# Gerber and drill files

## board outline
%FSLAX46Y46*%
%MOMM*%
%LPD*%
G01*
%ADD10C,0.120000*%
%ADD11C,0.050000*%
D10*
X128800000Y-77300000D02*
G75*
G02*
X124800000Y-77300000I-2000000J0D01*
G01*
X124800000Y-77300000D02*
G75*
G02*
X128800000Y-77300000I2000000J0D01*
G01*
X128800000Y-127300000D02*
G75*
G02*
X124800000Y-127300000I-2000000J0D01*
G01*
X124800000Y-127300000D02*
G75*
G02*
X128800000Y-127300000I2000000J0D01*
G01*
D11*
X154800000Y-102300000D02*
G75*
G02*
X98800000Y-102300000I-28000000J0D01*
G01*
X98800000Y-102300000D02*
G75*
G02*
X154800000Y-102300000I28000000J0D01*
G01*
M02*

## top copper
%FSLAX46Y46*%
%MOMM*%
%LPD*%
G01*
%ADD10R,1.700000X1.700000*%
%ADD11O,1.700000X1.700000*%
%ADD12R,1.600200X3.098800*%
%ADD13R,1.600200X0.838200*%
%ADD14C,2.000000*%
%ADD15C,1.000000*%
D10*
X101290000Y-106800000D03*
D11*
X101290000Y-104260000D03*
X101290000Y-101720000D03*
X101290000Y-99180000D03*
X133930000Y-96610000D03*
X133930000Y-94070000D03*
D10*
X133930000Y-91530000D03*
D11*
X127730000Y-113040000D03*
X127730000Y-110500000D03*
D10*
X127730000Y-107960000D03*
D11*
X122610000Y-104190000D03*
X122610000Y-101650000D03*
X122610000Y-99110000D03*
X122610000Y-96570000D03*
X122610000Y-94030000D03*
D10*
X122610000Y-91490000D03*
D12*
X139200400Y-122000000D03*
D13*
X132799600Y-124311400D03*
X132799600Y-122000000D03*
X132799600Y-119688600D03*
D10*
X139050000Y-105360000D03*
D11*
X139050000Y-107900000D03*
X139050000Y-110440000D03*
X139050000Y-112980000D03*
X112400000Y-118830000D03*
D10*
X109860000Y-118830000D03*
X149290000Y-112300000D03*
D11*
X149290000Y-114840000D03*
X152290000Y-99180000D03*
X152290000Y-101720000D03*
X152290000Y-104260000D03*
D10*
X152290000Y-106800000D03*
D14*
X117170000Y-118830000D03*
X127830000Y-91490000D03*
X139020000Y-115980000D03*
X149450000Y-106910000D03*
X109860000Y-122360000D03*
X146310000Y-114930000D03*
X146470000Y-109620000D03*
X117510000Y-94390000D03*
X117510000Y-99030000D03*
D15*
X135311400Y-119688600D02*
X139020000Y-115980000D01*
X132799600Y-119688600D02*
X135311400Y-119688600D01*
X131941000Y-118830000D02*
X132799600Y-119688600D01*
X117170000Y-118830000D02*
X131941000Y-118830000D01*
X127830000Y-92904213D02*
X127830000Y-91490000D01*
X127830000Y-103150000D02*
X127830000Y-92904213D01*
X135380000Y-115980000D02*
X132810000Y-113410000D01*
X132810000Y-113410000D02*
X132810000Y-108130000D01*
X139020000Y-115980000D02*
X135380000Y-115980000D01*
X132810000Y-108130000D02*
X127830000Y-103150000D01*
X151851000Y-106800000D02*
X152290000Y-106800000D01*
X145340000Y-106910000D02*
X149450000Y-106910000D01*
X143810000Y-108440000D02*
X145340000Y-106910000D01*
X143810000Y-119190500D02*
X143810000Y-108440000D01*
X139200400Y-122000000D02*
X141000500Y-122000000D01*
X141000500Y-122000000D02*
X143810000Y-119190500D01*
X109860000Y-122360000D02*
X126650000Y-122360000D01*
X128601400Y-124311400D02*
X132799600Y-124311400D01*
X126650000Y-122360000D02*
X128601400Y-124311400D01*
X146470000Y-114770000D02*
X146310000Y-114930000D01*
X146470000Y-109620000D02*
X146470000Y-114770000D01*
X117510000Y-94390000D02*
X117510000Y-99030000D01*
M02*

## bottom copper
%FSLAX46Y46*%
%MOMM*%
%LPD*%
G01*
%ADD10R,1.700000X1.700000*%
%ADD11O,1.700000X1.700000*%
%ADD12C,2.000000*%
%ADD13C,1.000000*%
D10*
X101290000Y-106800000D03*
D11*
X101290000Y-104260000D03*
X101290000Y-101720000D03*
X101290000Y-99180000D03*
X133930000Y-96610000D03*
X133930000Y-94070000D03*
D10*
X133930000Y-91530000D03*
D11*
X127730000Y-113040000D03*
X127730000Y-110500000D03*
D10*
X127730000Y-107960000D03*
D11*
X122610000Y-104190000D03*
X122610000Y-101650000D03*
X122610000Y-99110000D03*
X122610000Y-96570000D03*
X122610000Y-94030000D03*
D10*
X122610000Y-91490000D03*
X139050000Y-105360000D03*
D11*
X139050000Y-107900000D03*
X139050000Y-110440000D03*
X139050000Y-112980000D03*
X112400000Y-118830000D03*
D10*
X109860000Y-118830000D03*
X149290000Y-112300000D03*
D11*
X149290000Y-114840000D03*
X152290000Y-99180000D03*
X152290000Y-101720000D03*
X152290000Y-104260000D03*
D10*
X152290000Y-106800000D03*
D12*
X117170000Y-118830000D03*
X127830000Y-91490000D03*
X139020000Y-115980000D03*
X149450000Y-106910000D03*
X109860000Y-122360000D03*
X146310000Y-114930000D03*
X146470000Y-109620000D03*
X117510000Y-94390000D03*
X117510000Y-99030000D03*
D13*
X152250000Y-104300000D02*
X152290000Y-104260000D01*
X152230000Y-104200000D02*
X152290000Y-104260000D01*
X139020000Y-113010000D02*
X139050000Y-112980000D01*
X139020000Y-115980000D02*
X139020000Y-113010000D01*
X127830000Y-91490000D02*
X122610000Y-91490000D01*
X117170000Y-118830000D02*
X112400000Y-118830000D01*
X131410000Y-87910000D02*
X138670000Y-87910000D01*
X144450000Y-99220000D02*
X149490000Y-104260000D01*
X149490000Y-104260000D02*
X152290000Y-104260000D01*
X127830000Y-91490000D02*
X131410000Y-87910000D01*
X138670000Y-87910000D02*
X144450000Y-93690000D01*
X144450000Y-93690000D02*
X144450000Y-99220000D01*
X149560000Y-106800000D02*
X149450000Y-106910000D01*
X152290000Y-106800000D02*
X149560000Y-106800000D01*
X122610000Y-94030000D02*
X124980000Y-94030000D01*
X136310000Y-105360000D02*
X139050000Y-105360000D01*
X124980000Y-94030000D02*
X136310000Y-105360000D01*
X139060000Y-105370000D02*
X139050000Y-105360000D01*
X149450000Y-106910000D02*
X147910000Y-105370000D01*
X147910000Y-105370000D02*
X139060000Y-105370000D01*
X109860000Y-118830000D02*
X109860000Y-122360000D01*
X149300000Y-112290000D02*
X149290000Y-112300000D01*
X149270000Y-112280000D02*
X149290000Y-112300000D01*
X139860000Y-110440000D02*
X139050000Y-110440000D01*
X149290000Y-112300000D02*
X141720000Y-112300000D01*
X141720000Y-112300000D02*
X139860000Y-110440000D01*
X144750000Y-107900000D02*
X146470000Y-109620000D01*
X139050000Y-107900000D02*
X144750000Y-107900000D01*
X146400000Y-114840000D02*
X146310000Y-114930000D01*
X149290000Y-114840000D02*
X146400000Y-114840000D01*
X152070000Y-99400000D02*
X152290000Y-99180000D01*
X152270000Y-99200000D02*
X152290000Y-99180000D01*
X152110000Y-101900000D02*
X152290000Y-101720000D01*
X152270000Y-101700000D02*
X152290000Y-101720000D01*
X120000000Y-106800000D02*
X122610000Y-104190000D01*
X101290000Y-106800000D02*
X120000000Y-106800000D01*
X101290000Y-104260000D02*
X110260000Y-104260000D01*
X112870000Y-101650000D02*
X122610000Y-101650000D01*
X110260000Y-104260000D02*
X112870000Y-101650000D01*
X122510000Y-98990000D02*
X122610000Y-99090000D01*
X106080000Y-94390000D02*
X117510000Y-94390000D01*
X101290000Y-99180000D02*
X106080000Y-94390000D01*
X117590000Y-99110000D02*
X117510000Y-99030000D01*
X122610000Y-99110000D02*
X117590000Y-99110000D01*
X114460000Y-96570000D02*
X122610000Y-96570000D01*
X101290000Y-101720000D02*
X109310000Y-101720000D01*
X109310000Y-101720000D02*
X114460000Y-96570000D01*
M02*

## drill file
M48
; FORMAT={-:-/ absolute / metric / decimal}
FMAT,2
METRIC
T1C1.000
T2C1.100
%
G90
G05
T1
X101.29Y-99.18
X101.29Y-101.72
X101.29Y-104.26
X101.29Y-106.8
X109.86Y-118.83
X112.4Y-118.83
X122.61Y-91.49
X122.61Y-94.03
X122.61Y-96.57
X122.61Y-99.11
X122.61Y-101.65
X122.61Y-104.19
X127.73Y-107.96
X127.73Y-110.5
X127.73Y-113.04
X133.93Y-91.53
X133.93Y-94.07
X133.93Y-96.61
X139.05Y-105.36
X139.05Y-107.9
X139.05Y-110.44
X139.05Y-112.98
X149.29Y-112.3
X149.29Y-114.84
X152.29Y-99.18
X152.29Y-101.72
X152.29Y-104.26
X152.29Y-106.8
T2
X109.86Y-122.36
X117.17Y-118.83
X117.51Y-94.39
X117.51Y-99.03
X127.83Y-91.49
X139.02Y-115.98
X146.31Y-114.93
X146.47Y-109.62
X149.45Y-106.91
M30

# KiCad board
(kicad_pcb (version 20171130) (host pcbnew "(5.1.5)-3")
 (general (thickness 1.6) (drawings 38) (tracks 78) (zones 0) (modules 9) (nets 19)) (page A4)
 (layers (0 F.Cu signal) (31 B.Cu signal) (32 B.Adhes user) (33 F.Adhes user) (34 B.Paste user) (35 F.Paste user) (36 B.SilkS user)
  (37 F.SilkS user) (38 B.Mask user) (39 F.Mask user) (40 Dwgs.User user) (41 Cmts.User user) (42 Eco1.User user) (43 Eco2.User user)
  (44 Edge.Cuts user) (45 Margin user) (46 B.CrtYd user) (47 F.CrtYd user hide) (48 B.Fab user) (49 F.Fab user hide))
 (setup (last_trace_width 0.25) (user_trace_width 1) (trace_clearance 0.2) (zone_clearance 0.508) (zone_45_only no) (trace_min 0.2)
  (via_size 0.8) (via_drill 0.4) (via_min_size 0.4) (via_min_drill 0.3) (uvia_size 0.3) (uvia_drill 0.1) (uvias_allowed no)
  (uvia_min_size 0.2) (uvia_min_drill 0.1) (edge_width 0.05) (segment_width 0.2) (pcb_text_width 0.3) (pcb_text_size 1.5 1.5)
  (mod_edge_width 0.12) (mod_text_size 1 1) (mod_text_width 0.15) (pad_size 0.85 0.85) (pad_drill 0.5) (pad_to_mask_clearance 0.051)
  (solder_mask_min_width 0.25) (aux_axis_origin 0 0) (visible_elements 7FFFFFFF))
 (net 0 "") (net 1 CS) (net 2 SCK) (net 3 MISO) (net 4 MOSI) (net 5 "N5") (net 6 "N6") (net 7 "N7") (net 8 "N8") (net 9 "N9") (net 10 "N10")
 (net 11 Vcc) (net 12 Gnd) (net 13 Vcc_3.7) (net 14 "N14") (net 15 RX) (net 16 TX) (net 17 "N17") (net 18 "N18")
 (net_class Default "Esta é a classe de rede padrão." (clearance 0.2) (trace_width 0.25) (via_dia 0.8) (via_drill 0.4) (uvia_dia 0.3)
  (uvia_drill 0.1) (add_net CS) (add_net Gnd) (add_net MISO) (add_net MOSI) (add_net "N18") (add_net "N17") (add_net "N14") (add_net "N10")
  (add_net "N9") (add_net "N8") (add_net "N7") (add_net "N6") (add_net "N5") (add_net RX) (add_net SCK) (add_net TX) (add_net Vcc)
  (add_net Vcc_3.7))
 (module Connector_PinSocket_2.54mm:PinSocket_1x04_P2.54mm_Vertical (layer F.Cu) (at 101.29 106.8 180)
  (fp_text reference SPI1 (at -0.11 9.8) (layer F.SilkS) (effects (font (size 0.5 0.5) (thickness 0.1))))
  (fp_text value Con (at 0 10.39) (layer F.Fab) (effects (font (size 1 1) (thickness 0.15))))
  (pad 1 thru_hole rect (at 0 0 180) (size 1.7 1.7) (drill 1) (layers *.Cu *.Mask) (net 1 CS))
  (pad 2 thru_hole oval (at 0 2.54 180) (size 1.7 1.7) (drill 1) (layers *.Cu *.Mask) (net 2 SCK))
  (pad 3 thru_hole oval (at 0 5.08 180) (size 1.7 1.7) (drill 1) (layers *.Cu *.Mask) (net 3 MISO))
  (pad 4 thru_hole oval (at 0 7.62 180) (size 1.7 1.7) (drill 1) (layers *.Cu *.Mask) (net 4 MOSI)))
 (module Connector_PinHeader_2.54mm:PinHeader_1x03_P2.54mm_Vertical (layer F.Cu) (at 133.93 91.53)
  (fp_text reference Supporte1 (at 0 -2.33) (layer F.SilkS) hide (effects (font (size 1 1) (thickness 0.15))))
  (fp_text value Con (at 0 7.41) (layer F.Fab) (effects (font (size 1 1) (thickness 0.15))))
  (pad 3 thru_hole oval (at 0 5.08) (size 1.7 1.7) (drill 1) (layers *.Cu *.Mask) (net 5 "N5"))
  (pad 2 thru_hole oval (at 0 2.54) (size 1.7 1.7) (drill 1) (layers *.Cu *.Mask) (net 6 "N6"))
  (pad 1 thru_hole rect (at 0 0) (size 1.7 1.7) (drill 1) (layers *.Cu *.Mask) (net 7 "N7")))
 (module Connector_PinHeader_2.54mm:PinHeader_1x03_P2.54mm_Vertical (layer F.Cu) (at 127.73 107.96)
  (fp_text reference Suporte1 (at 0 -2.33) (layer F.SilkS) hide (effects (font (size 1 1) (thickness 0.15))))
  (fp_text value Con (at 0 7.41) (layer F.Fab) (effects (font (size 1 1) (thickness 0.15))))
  (pad 3 thru_hole oval (at 0 5.08) (size 1.7 1.7) (drill 1) (layers *.Cu *.Mask) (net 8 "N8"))
  (pad 2 thru_hole oval (at 0 2.54) (size 1.7 1.7) (drill 1) (layers *.Cu *.Mask) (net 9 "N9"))
  (pad 1 thru_hole rect (at 0 0) (size 1.7 1.7) (drill 1) (layers *.Cu *.Mask) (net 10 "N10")))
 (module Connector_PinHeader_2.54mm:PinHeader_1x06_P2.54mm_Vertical (layer F.Cu) (at 122.61 91.49)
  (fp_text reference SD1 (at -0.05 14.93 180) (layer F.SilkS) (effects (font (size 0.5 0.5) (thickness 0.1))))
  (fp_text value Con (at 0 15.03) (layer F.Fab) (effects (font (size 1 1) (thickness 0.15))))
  (pad 6 thru_hole oval (at 0 12.7) (size 1.7 1.7) (drill 1) (layers *.Cu *.Mask) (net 1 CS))
  (pad 5 thru_hole oval (at 0 10.16) (size 1.7 1.7) (drill 1) (layers *.Cu *.Mask) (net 2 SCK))
  (pad 4 thru_hole oval (at 0 7.62) (size 1.7 1.7) (drill 1) (layers *.Cu *.Mask) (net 4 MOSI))
  (pad 3 thru_hole oval (at 0 5.08) (size 1.7 1.7) (drill 1) (layers *.Cu *.Mask) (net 3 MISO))
  (pad 2 thru_hole oval (at 0 2.54) (size 1.7 1.7) (drill 1) (layers *.Cu *.Mask) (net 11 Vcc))
  (pad 1 thru_hole rect (at 0 0) (size 1.7 1.7) (drill 1) (layers *.Cu *.Mask) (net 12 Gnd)))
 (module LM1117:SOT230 (layer F.Cu) (at 136 122)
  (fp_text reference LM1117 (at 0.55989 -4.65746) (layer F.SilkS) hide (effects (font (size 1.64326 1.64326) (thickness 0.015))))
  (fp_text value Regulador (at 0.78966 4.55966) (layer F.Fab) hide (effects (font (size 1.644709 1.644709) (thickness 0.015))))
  (pad 4 smd rect (at 3.2004 0) (size 1.6002 3.0988) (layers F.Cu F.Paste F.Mask) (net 11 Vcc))
  (pad 3 smd rect (at -3.2004 2.3114) (size 1.6002 0.8382) (layers F.Cu F.Paste F.Mask) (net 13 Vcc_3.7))
  (pad 2 smd rect (at -3.2004 0) (size 1.6002 0.8382) (layers F.Cu F.Paste F.Mask) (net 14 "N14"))
  (pad 1 smd rect (at -3.2004 -2.3114) (size 1.6002 0.8382) (layers F.Cu F.Paste F.Mask) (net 12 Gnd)))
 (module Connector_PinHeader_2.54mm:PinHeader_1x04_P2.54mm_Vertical (layer F.Cu) (at 139.05 105.36)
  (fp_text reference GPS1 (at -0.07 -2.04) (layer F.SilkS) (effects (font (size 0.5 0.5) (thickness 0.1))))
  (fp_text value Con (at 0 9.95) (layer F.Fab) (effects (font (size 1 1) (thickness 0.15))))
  (pad 1 thru_hole rect (at 0 0) (size 1.7 1.7) (drill 1) (layers *.Cu *.Mask) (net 11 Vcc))
  (pad 2 thru_hole oval (at 0 2.54) (size 1.7 1.7) (drill 1) (layers *.Cu *.Mask) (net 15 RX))
  (pad 3 thru_hole oval (at 0 5.08) (size 1.7 1.7) (drill 1) (layers *.Cu *.Mask) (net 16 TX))
  (pad 4 thru_hole oval (at 0 7.62) (size 1.7 1.7) (drill 1) (layers *.Cu *.Mask) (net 12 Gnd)))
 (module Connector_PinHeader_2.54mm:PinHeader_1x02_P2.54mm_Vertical (layer F.Cu) (at 109.86 118.83 90)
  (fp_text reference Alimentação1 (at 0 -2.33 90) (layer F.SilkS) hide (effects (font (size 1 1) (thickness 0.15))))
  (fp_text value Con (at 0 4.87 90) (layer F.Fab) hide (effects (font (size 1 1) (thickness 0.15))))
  (pad 2 thru_hole oval (at 0 2.54 90) (size 1.7 1.7) (drill 1) (layers *.Cu *.Mask) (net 12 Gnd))
  (pad 1 thru_hole rect (at 0 0 90) (size 1.7 1.7) (drill 1) (layers *.Cu *.Mask) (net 13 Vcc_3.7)))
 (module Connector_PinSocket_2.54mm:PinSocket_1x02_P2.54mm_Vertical (layer F.Cu) (at 149.29 112.3)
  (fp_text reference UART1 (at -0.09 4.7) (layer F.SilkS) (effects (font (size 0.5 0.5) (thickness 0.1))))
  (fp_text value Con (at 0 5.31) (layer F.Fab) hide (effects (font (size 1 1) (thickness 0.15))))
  (pad 1 thru_hole rect (at 0 0) (size 1.7 1.7) (drill 1) (layers *.Cu *.Mask) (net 16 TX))
  (pad 2 thru_hole oval (at 0 2.54) (size 1.7 1.7) (drill 1) (layers *.Cu *.Mask) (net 15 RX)))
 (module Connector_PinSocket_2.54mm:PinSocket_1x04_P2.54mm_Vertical (layer F.Cu) (at 152.29 106.8 180)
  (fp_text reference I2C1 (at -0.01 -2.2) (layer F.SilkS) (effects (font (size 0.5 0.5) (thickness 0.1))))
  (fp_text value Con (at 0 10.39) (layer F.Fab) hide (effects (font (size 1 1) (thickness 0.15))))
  (pad 4 thru_hole oval (at 0 7.62 180) (size 1.7 1.7) (drill 1) (layers *.Cu *.Mask) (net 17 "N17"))
  (pad 3 thru_hole oval (at 0 5.08 180) (size 1.7 1.7) (drill 1) (layers *.Cu *.Mask) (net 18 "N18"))
  (pad 2 thru_hole oval (at 0 2.54 180) (size 1.7 1.7) (drill 1) (layers *.Cu *.Mask) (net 12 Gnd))
  (pad 1 thru_hole rect (at 0 0 180) (size 1.7 1.7) (drill 1) (layers *.Cu *.Mask) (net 11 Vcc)))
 (gr_circle (center 126.8 77.3) (end 128.8 77.3) (layer Edge.Cuts) (width 0.12))
 (gr_circle (center 126.8 127.3) (end 128.8 127.3) (layer Edge.Cuts) (width 0.12))
 (gr_circle (center 126.8 102.3) (end 154.8 102.3) (layer Edge.Cuts) (width 0.05))
 (via (at 117.17 118.83) (size 2) (drill 1.1) (layers F.Cu B.Cu) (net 12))
 (via (at 127.83 91.49) (size 2) (drill 1.1) (layers F.Cu B.Cu) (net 12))
 (via (at 139.02 115.98) (size 2) (drill 1.1) (layers F.Cu B.Cu) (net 12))
 (segment (start 152.25 104.3) (end 152.29 104.26) (width 1) (layer B.Cu) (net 12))
 (segment (start 152.23 104.2) (end 152.29 104.26) (width 1) (layer B.Cu) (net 12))
 (segment (start 135.3114 119.6886) (end 139.02 115.98) (width 1) (layer F.Cu) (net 12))
 (segment (start 132.7996 119.6886) (end 135.3114 119.6886) (width 1) (layer F.Cu) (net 12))
 (segment (start 139.02 113.01) (end 139.05 112.98) (width 1) (layer B.Cu) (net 12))
 (segment (start 139.02 115.98) (end 139.02 113.01) (width 1) (layer B.Cu) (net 12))
 (segment (start 127.83 91.49) (end 122.61 91.49) (width 1) (layer B.Cu) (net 12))
 (segment (start 117.17 118.83) (end 112.4 118.83) (width 1) (layer B.Cu) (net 12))
 (segment (start 131.941 118.83) (end 132.7996 119.6886) (width 1) (layer F.Cu) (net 12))
 (segment (start 117.17 118.83) (end 131.941 118.83) (width 1) (layer F.Cu) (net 12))
 (segment (start 131.41 87.91) (end 138.67 87.91) (width 1) (layer B.Cu) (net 12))
 (segment (start 144.45 99.22) (end 149.49 104.26) (width 1) (layer B.Cu) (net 12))
 (segment (start 149.49 104.26) (end 152.29 104.26) (width 1) (layer B.Cu) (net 12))
 (segment (start 127.83 91.49) (end 131.41 87.91) (width 1) (layer B.Cu) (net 12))
 (segment (start 138.67 87.91) (end 144.45 93.69) (width 1) (layer B.Cu) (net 12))
 (segment (start 144.45 93.69) (end 144.45 99.22) (width 1) (layer B.Cu) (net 12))
 (segment (start 127.83 92.904213) (end 127.83 91.49) (width 1) (layer F.Cu) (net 12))
 (segment (start 127.83 103.15) (end 127.83 92.904213) (width 1) (layer F.Cu) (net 12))
 (segment (start 135.38 115.98) (end 132.81 113.41) (width 1) (layer F.Cu) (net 12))
 (segment (start 132.81 113.41) (end 132.81 108.13) (width 1) (layer F.Cu) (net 12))
 (segment (start 139.02 115.98) (end 135.38 115.98) (width 1) (layer F.Cu) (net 12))
 (segment (start 132.81 108.13) (end 127.83 103.15) (width 1) (layer F.Cu) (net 12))
 (via (at 149.45 106.91) (size 2) (drill 1.1) (layers F.Cu B.Cu) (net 11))
 (segment (start 151.851 106.8) (end 152.29 106.8) (width 1) (layer F.Cu) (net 11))
 (segment (start 149.56 106.8) (end 149.45 106.91) (width 1) (layer B.Cu) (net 11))
 (segment (start 152.29 106.8) (end 149.56 106.8) (width 1) (layer B.Cu) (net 11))
 (segment (start 122.61 94.03) (end 124.98 94.03) (width 1) (layer B.Cu) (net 11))
 (segment (start 136.31 105.36) (end 139.05 105.36) (width 1) (layer B.Cu) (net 11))
 (segment (start 124.98 94.03) (end 136.31 105.36) (width 1) (layer B.Cu) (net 11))
 (segment (start 139.06 105.37) (end 139.05 105.36) (width 1) (layer B.Cu) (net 11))
 (segment (start 149.45 106.91) (end 147.91 105.37) (width 1) (layer B.Cu) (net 11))
 (segment (start 147.91 105.37) (end 139.06 105.37) (width 1) (layer B.Cu) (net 11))
 (segment (start 145.34 106.91) (end 149.45 106.91) (width 1) (layer F.Cu) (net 11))
 (segment (start 143.81 108.44) (end 145.34 106.91) (width 1) (layer F.Cu) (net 11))
 (segment (start 143.81 119.1905) (end 143.81 108.44) (width 1) (layer F.Cu) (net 11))
 (segment (start 139.2004 122) (end 141.0005 122) (width 1) (layer F.Cu) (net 11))
 (segment (start 141.0005 122) (end 143.81 119.1905) (width 1) (layer F.Cu) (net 11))
 (via (at 109.86 122.36) (size 2) (drill 1.1) (layers F.Cu B.Cu) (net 13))
 (segment (start 109.86 118.83) (end 109.86 122.36) (width 1) (layer B.Cu) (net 13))
 (segment (start 109.86 122.36) (end 126.65 122.36) (width 1) (layer F.Cu) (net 13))
 (segment (start 128.6014 124.3114) (end 132.7996 124.3114) (width 1) (layer F.Cu) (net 13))
 (segment (start 126.65 122.36) (end 128.6014 124.3114) (width 1) (layer F.Cu) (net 13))
 (segment (start 149.3 112.29) (end 149.29 112.3) (width 1) (layer B.Cu) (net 16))
 (segment (start 149.27 112.28) (end 149.29 112.3) (width 1) (layer B.Cu) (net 16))
 (segment (start 139.86 110.44) (end 139.05 110.44) (width 1) (layer B.Cu) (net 16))
 (segment (start 149.29 112.3) (end 141.72 112.3) (width 1) (layer B.Cu) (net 16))
 (segment (start 141.72 112.3) (end 139.86 110.44) (width 1) (layer B.Cu) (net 16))
 (via (at 146.31 114.93) (size 2) (drill 1.1) (layers F.Cu B.Cu) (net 15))
 (via (at 146.47 109.62) (size 2) (drill 1.1) (layers F.Cu B.Cu) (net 15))
 (segment (start 144.75 107.9) (end 146.47 109.62) (width 1) (layer B.Cu) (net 15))
 (segment (start 139.05 107.9) (end 144.75 107.9) (width 1) (layer B.Cu) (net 15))
 (segment (start 146.47 114.77) (end 146.31 114.93) (width 1) (layer F.Cu) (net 15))
 (segment (start 146.47 109.62) (end 146.47 114.77) (width 1) (layer F.Cu) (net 15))
 (segment (start 146.4 114.84) (end 146.31 114.93) (width 1) (layer B.Cu) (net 15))
 (segment (start 149.29 114.84) (end 146.4 114.84) (width 1) (layer B.Cu) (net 15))
 (segment (start 152.07 99.4) (end 152.29 99.18) (width 1) (layer B.Cu) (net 17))
 (segment (start 152.27 99.2) (end 152.29 99.18) (width 1) (layer B.Cu) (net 17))
 (segment (start 152.11 101.9) (end 152.29 101.72) (width 1) (layer B.Cu) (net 18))
 (segment (start 152.27 101.7) (end 152.29 101.72) (width 1) (layer B.Cu) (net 18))
 (segment (start 120 106.8) (end 122.61 104.19) (width 1) (layer B.Cu) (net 1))
 (segment (start 101.29 106.8) (end 120 106.8) (width 1) (layer B.Cu) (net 1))
 (segment (start 101.29 104.26) (end 110.26 104.26) (width 1) (layer B.Cu) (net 2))
 (segment (start 112.87 101.65) (end 122.61 101.65) (width 1) (layer B.Cu) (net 2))
 (segment (start 110.26 104.26) (end 112.87 101.65) (width 1) (layer B.Cu) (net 2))
 (via (at 117.51 94.39) (size 2) (drill 1.1) (layers F.Cu B.Cu) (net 4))
 (via (at 117.51 99.03) (size 2) (drill 1.1) (layers F.Cu B.Cu) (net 4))
 (segment (start 122.51 98.99) (end 122.61 99.09) (width 1) (layer B.Cu) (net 4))
 (segment (start 106.08 94.39) (end 117.51 94.39) (width 1) (layer B.Cu) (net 4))
 (segment (start 101.29 99.18) (end 106.08 94.39) (width 1) (layer B.Cu) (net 4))
 (segment (start 117.51 94.39) (end 117.51 99.03) (width 1) (layer F.Cu) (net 4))
 (segment (start 117.59 99.11) (end 117.51 99.03) (width 1) (layer B.Cu) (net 4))
 (segment (start 122.61 99.11) (end 117.59 99.11) (width 1) (layer B.Cu) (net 4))
 (segment (start 114.46 96.57) (end 122.61 96.57) (width 1) (layer B.Cu) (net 3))
 (segment (start 101.29 101.72) (end 109.31 101.72) (width 1) (layer B.Cu) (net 3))
 (segment (start 109.31 101.72) (end 114.46 96.57) (width 1) (layer B.Cu) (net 3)))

